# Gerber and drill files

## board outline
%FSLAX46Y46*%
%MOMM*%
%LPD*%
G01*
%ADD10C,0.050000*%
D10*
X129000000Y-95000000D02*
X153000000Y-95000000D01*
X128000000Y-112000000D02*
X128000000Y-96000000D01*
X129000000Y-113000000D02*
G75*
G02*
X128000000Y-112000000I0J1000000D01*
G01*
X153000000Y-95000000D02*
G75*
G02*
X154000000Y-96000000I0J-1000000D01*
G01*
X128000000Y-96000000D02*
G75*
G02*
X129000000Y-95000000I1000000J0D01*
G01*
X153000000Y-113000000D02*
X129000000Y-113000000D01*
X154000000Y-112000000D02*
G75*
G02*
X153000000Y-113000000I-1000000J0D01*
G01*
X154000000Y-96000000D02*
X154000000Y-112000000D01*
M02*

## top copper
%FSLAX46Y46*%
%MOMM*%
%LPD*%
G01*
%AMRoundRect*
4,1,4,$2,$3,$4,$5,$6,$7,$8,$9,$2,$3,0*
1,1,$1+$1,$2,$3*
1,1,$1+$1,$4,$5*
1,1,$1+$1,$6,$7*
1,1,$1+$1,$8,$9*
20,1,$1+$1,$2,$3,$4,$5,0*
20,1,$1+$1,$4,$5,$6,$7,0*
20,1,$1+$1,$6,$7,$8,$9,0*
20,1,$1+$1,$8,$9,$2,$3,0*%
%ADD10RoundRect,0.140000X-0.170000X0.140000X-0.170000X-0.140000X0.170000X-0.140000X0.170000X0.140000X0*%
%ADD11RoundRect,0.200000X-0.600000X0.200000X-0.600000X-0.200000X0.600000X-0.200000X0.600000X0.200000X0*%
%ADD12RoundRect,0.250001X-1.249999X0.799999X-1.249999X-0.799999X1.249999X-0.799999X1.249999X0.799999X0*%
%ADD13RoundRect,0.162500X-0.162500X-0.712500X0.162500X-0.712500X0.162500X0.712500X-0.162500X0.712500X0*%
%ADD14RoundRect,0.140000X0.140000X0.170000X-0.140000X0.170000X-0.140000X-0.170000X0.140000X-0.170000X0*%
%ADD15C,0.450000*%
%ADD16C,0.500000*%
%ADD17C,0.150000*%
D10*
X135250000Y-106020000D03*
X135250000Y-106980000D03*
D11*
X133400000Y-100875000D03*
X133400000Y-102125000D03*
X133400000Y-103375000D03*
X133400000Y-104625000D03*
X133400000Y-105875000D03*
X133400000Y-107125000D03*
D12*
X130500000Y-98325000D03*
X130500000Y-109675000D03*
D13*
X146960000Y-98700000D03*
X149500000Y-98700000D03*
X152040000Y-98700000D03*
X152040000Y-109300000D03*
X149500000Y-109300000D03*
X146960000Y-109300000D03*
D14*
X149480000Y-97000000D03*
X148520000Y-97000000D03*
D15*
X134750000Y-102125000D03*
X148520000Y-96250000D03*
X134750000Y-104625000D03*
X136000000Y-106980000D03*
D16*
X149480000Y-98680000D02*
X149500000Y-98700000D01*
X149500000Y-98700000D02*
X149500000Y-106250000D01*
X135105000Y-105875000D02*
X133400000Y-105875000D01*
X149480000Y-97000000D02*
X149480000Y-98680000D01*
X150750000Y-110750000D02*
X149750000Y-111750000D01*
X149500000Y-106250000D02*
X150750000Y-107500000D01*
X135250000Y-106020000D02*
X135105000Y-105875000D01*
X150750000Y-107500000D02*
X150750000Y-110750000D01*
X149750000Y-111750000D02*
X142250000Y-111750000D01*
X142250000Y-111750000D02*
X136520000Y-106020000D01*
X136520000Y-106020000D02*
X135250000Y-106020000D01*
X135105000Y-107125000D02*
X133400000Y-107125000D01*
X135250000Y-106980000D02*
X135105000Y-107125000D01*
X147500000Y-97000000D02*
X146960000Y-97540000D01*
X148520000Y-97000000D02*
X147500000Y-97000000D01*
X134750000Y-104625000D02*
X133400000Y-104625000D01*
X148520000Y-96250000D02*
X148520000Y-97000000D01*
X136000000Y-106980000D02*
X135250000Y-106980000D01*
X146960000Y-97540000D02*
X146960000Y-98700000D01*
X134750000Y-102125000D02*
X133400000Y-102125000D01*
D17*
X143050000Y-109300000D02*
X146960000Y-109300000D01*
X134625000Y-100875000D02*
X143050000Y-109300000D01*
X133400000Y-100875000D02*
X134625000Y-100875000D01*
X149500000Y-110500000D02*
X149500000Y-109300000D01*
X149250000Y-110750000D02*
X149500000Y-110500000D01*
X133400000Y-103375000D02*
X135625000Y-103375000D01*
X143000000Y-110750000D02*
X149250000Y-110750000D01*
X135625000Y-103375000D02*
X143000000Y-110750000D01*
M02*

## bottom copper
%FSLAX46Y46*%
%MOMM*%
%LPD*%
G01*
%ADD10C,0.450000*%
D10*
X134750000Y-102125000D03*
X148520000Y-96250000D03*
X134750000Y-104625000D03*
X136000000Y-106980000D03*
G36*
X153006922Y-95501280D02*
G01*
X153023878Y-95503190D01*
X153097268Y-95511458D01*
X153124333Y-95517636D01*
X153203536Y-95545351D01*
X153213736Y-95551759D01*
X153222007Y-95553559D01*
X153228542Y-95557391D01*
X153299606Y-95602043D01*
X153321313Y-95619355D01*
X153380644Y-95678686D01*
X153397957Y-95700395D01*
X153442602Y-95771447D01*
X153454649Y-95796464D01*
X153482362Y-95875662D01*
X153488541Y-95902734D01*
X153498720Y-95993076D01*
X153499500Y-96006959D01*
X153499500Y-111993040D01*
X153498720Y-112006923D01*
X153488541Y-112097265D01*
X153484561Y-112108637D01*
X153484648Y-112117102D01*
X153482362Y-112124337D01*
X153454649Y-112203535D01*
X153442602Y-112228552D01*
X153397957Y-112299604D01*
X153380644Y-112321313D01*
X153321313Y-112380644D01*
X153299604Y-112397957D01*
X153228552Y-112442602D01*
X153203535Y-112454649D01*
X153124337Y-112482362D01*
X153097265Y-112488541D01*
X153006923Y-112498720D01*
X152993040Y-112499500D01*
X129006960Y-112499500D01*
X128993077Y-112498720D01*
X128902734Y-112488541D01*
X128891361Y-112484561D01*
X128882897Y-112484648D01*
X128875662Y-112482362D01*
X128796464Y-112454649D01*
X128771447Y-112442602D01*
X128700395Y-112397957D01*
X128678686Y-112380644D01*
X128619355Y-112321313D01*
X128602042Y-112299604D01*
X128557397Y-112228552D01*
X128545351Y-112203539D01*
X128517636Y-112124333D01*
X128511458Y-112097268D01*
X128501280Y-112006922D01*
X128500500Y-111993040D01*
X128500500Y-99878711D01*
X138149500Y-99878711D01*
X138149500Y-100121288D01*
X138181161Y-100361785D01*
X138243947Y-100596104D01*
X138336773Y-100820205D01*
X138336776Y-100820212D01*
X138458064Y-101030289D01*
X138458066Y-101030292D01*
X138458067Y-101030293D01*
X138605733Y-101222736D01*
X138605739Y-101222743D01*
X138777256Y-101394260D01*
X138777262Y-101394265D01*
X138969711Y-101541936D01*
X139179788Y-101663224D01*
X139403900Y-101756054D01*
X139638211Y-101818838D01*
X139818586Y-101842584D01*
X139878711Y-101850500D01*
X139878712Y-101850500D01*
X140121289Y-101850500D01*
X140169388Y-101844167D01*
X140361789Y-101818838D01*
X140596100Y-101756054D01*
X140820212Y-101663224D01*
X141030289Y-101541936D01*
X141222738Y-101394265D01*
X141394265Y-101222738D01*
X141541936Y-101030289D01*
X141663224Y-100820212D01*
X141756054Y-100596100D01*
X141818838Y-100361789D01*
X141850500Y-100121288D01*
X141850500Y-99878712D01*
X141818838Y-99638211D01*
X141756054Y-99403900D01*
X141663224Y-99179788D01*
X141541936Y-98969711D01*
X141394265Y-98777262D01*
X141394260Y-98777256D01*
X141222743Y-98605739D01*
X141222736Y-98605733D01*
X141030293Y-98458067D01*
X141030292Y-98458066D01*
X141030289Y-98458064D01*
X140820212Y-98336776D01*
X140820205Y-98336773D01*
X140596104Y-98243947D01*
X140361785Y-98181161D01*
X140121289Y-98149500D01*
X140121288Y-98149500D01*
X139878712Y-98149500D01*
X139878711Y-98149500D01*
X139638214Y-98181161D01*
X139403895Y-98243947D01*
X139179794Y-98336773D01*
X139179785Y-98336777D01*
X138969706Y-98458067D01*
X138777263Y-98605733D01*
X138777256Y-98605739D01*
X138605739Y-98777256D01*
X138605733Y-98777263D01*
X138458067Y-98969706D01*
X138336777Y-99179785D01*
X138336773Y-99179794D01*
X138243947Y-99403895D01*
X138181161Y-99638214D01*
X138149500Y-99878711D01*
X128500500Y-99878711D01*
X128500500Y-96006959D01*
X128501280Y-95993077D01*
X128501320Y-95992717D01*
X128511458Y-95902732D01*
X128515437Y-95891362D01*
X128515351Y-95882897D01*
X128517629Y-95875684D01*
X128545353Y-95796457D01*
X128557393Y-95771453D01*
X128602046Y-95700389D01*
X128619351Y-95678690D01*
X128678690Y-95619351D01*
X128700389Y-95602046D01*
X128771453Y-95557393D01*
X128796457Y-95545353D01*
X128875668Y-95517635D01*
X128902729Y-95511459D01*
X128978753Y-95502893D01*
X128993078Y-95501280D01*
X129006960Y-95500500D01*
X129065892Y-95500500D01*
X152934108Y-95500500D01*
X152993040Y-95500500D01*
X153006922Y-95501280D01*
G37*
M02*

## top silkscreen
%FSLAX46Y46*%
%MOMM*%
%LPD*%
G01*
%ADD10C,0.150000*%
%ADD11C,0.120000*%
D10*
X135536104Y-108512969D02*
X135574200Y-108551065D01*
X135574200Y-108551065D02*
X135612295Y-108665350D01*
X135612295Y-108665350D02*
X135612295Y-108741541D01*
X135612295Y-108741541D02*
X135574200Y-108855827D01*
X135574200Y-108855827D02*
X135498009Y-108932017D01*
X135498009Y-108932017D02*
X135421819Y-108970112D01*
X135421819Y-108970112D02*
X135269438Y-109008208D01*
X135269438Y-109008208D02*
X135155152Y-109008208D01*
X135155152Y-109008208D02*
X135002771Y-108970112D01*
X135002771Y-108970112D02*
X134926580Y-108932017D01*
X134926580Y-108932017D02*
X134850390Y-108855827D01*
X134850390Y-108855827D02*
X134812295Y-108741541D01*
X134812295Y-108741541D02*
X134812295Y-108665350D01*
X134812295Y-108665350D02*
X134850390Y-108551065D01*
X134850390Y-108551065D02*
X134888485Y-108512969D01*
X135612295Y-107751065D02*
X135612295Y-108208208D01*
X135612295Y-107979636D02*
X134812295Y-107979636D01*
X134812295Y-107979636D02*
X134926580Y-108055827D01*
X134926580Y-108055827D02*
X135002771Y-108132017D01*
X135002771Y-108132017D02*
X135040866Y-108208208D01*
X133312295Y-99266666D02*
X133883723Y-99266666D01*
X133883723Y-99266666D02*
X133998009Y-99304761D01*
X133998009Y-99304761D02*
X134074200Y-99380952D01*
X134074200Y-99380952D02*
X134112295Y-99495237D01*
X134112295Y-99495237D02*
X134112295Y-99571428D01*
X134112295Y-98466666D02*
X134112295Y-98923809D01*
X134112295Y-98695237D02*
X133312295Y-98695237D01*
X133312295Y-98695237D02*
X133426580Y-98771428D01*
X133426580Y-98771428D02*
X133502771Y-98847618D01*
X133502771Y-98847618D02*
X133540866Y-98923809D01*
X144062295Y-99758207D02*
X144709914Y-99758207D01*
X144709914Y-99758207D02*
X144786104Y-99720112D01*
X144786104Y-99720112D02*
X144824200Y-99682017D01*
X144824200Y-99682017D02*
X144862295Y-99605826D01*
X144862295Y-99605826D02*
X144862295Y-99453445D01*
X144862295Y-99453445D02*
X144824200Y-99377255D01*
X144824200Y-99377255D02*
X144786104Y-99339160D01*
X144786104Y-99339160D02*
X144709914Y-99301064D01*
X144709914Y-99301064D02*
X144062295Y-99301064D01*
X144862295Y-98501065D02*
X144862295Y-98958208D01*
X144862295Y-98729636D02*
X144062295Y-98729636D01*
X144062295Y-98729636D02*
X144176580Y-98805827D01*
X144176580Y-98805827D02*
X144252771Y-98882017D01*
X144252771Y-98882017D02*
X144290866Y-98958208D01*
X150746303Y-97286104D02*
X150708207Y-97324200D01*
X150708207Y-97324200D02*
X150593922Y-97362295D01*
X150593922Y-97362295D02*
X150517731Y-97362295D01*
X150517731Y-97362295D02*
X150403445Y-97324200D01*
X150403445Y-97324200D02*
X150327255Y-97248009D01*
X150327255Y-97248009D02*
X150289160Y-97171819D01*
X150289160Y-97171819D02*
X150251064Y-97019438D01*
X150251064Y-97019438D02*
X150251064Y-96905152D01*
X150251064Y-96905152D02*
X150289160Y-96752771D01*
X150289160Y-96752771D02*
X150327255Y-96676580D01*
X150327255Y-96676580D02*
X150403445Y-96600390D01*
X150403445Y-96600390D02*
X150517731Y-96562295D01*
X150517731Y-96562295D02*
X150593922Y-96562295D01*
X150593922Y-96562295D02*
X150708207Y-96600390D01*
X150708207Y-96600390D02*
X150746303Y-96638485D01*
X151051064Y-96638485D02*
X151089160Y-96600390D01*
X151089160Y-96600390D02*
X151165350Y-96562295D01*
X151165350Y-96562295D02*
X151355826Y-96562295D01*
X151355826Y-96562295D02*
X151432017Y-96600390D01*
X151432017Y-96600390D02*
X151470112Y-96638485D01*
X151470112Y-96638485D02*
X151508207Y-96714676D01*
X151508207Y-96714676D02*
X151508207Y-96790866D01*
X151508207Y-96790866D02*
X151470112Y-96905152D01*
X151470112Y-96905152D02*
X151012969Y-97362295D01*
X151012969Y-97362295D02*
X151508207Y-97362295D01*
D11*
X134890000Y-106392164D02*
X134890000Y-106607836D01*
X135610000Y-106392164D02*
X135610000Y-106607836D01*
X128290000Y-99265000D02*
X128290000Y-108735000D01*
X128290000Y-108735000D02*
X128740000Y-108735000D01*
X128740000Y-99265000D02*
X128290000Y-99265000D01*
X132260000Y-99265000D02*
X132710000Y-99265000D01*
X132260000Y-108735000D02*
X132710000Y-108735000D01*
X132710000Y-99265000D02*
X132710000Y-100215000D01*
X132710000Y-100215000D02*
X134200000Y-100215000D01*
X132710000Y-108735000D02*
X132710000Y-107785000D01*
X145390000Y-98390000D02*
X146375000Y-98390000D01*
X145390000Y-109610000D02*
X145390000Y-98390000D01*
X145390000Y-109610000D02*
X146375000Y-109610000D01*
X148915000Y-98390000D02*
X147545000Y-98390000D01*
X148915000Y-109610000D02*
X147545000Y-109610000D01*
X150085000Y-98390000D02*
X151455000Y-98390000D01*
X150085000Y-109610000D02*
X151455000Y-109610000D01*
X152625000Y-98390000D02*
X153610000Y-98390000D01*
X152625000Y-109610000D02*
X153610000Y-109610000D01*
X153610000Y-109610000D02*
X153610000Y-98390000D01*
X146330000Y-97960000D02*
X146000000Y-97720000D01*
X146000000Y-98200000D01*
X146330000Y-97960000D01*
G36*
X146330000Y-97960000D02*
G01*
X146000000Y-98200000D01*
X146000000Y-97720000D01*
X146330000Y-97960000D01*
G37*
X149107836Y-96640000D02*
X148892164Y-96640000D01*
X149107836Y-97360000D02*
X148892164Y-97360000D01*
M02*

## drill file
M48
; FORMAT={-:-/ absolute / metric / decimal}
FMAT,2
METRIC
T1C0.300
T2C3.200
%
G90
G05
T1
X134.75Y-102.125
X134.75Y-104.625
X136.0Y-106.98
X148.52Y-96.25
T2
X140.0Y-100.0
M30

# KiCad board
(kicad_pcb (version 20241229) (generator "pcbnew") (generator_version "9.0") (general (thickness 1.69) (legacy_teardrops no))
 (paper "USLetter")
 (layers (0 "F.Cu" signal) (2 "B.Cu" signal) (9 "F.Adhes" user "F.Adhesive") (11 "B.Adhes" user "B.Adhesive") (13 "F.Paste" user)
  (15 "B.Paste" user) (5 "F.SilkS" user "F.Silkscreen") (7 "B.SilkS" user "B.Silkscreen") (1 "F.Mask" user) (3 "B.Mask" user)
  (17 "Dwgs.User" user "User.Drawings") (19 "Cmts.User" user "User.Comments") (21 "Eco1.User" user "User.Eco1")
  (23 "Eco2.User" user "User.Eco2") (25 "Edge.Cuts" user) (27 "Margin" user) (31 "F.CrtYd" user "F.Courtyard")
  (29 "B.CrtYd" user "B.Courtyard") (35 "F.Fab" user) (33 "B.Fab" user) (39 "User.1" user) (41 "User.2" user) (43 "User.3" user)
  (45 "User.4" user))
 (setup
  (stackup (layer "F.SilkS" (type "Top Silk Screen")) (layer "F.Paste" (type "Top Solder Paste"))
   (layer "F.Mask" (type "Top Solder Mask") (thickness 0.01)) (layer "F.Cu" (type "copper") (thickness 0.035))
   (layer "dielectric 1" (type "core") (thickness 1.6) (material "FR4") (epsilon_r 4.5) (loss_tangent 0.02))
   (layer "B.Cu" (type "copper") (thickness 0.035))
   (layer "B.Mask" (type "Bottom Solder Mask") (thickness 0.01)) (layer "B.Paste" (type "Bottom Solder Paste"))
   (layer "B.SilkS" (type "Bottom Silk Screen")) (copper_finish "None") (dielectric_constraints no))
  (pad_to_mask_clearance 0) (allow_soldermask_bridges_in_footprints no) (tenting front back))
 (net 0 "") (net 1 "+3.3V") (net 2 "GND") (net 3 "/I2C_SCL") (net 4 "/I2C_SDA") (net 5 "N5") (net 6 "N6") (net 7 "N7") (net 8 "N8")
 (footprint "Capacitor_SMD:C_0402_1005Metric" (layer "F.Cu") (at 135.25 106.5 -90)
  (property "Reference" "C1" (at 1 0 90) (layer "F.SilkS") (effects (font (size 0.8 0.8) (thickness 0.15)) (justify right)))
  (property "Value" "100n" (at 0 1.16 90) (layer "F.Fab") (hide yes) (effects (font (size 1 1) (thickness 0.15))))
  (fp_line (start -0.107836 0.36) (end 0.107836 0.36) (stroke (width 0.12) (type solid)) (layer "F.SilkS"))
  (fp_line (start -0.107836 -0.36) (end 0.107836 -0.36) (stroke (width 0.12) (type solid)) (layer "F.SilkS"))
  (pad "1" smd roundrect (at -0.48 0 270) (size 0.56 0.62) (layers "F.Cu" "F.Mask" "F.Paste") (roundrect_rratio 0.25) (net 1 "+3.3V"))
  (pad "2" smd roundrect (at 0.48 0 270) (size 0.56 0.62) (layers "F.Cu" "F.Mask" "F.Paste") (roundrect_rratio 0.25) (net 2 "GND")))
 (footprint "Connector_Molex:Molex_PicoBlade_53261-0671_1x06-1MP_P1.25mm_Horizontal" (layer "F.Cu") (at 131 104 -90)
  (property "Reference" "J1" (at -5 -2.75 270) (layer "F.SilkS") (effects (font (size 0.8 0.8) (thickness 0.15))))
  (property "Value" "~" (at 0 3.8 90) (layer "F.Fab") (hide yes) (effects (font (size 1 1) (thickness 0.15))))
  (fp_line (start -4.735 2.71) (end 4.735 2.71) (stroke (width 0.12) (type solid)) (layer "F.SilkS"))
  (fp_line (start 4.735 2.71) (end 4.735 2.26) (stroke (width 0.12) (type solid)) (layer "F.SilkS"))
  (fp_line (start -4.735 2.26) (end -4.735 2.71) (stroke (width 0.12) (type solid)) (layer "F.SilkS"))
  (fp_line (start -4.735 -1.26) (end -4.735 -1.71) (stroke (width 0.12) (type solid)) (layer "F.SilkS"))
  (fp_line (start 4.735 -1.26) (end 4.735 -1.71) (stroke (width 0.12) (type solid)) (layer "F.SilkS"))
  (fp_line (start -4.735 -1.71) (end -3.785 -1.71) (stroke (width 0.12) (type solid)) (layer "F.SilkS"))
  (fp_line (start -3.785 -1.71) (end -3.785 -3.2) (stroke (width 0.12) (type solid)) (layer "F.SilkS"))
  (fp_line (start 4.735 -1.71) (end 3.785 -1.71) (stroke (width 0.12) (type solid)) (layer "F.SilkS"))
  (pad "1" smd roundrect (at -3.125 -2.4 270) (size 0.8 1.6) (layers "F.Cu" "F.Mask" "F.Paste") (roundrect_rratio 0.25) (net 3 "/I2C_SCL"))
  (pad "2" smd roundrect (at -1.875 -2.4 270) (size 0.8 1.6) (layers "F.Cu" "F.Mask" "F.Paste") (roundrect_rratio 0.25) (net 2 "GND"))
  (pad "3" smd roundrect (at -0.625 -2.4 270) (size 0.8 1.6) (layers "F.Cu" "F.Mask" "F.Paste") (roundrect_rratio 0.25) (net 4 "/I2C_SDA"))
  (pad "4" smd roundrect (at 0.625 -2.4 270) (size 0.8 1.6) (layers "F.Cu" "F.Mask" "F.Paste") (roundrect_rratio 0.25) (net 2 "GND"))
  (pad "5" smd roundrect (at 1.875 -2.4 270) (size 0.8 1.6) (layers "F.Cu" "F.Mask" "F.Paste") (roundrect_rratio 0.25) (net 1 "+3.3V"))
  (pad "6" smd roundrect (at 3.125 -2.4 270) (size 0.8 1.6) (layers "F.Cu" "F.Mask" "F.Paste") (roundrect_rratio 0.25) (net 2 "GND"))
  (pad "MP" smd roundrect (at -5.675 0.5 270) (size 2.1 3) (layers "F.Cu" "F.Mask" "F.Paste") (roundrect_rratio 0.119048) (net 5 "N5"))
  (pad "MP" smd roundrect (at 5.675 0.5 270) (size 2.1 3) (layers "F.Cu" "F.Mask" "F.Paste") (roundrect_rratio 0.119048) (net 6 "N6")))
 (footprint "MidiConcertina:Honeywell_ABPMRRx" (layer "F.Cu") (at 149.5 104)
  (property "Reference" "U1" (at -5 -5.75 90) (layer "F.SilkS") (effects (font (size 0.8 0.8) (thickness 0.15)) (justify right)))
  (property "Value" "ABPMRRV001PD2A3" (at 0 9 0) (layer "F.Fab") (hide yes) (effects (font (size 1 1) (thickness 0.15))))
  (fp_line (start -4.11 -5.61) (end -3.125 -5.61) (stroke (width 0.12) (type solid)) (layer "F.SilkS"))
  (fp_line (start -4.11 5.61) (end -4.11 -5.61) (stroke (width 0.12) (type solid)) (layer "F.SilkS"))
  (fp_line (start -4.11 5.61) (end -3.125 5.61) (stroke (width 0.12) (type solid)) (layer "F.SilkS"))
  (fp_line (start -0.585 -5.61) (end -1.955 -5.61) (stroke (width 0.12) (type solid)) (layer "F.SilkS"))
  (fp_line (start -0.585 5.61) (end -1.955 5.61) (stroke (width 0.12) (type solid)) (layer "F.SilkS"))
  (fp_line (start 0.585 -5.61) (end 1.955 -5.61) (stroke (width 0.12) (type solid)) (layer "F.SilkS"))
  (fp_line (start 0.585 5.61) (end 1.955 5.61) (stroke (width 0.12) (type solid)) (layer "F.SilkS"))
  (fp_line (start 3.125 -5.61) (end 4.11 -5.61) (stroke (width 0.12) (type solid)) (layer "F.SilkS"))
  (fp_line (start 3.125 5.61) (end 4.11 5.61) (stroke (width 0.12) (type solid)) (layer "F.SilkS"))
  (fp_line (start 4.11 5.61) (end 4.11 -5.61) (stroke (width 0.12) (type solid)) (layer "F.SilkS"))
  (fp_poly
   (pts (xy -3.17 -6.04) (xy -3.5 -6.28) (xy -3.5 -5.8) (xy -3.17 -6.04)) (stroke (width 0.12) (type solid)) (fill yes) (layer "F.SilkS"))
  (pad "1" smd roundrect (at -2.54 -5.3) (size 0.65 1.75) (layers "F.Cu" "F.Mask" "F.Paste") (roundrect_rratio 0.25) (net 2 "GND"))
  (pad "2" smd roundrect (at 0 -5.3) (size 0.65 1.75) (layers "F.Cu" "F.Mask" "F.Paste") (roundrect_rratio 0.25) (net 1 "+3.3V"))
  (pad "3" smd roundrect (at 2.54 -5.3) (size 0.65 1.75) (layers "F.Cu" "F.Mask" "F.Paste") (roundrect_rratio 0.25) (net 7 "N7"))
  (pad "4" smd roundrect (at 2.54 5.3) (size 0.65 1.75) (layers "F.Cu" "F.Mask" "F.Paste") (roundrect_rratio 0.25) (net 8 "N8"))
  (pad "5" smd roundrect (at 0 5.3) (size 0.65 1.75) (layers "F.Cu" "F.Mask" "F.Paste") (roundrect_rratio 0.25) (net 4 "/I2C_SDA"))
  (pad "6" smd roundrect (at -2.54 5.3) (size 0.65 1.75) (layers "F.Cu" "F.Mask" "F.Paste") (roundrect_rratio 0.25) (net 3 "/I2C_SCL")))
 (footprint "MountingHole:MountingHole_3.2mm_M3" (layer "F.Cu") (at 140 100)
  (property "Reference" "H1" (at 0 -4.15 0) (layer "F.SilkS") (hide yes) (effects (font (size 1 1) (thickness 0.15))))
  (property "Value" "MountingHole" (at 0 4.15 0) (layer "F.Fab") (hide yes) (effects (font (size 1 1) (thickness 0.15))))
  (pad "" np_thru_hole circle (at 0 0) (size 3.2 3.2) (drill 3.2) (layers "*.Cu" "*.Mask")))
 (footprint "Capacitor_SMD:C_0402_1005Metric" (layer "F.Cu") (at 149 97 180)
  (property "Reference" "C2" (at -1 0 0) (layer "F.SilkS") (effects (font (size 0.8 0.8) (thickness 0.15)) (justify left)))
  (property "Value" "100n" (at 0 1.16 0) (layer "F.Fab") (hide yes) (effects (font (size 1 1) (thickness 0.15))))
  (fp_line (start -0.107836 0.36) (end 0.107836 0.36) (stroke (width 0.12) (type solid)) (layer "F.SilkS"))
  (fp_line (start -0.107836 -0.36) (end 0.107836 -0.36) (stroke (width 0.12) (type solid)) (layer "F.SilkS"))
  (pad "1" smd roundrect (at -0.48 0 180) (size 0.56 0.62) (layers "F.Cu" "F.Mask" "F.Paste") (roundrect_rratio 0.25) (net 1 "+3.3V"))
  (pad "2" smd roundrect (at 0.48 0 180) (size 0.56 0.62) (layers "F.Cu" "F.Mask" "F.Paste") (roundrect_rratio 0.25) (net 2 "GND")))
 (gr_line (start 129 95) (end 153 95) (stroke (width 0.05) (type default)) (layer "Edge.Cuts"))
 (gr_line (start 128 112) (end 128 96) (stroke (width 0.05) (type default)) (layer "Edge.Cuts"))
 (gr_arc (start 129 113) (mid 128.292893 112.707107) (end 128 112) (stroke (width 0.05) (type default)) (layer "Edge.Cuts"))
 (gr_arc (start 153 95) (mid 153.707107 95.292893) (end 154 96) (stroke (width 0.05) (type default)) (layer "Edge.Cuts"))
 (gr_arc (start 128 96) (mid 128.292893 95.292893) (end 129 95) (stroke (width 0.05) (type default)) (layer "Edge.Cuts"))
 (gr_line (start 153 113) (end 129 113) (stroke (width 0.05) (type default)) (layer "Edge.Cuts"))
 (gr_arc (start 154 112) (mid 153.707107 112.707107) (end 153 113) (stroke (width 0.05) (type default)) (layer "Edge.Cuts"))
 (gr_line (start 154 96) (end 154 112) (stroke (width 0.05) (type default)) (layer "Edge.Cuts"))
 (segment (start 149.48 98.68) (end 149.5 98.7) (width 0.5) (layer "F.Cu") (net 1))
 (segment (start 149.5 98.7) (end 149.5 106.25) (width 0.5) (layer "F.Cu") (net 1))
 (segment (start 135.105 105.875) (end 133.4 105.875) (width 0.5) (layer "F.Cu") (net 1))
 (segment (start 149.48 97) (end 149.48 98.68) (width 0.5) (layer "F.Cu") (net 1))
 (segment (start 150.75 110.75) (end 149.75 111.75) (width 0.5) (layer "F.Cu") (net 1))
 (segment (start 149.5 106.25) (end 150.75 107.5) (width 0.5) (layer "F.Cu") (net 1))
 (segment (start 135.25 106.02) (end 135.105 105.875) (width 0.5) (layer "F.Cu") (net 1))
 (segment (start 150.75 107.5) (end 150.75 110.75) (width 0.5) (layer "F.Cu") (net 1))
 (segment (start 149.75 111.75) (end 142.25 111.75) (width 0.5) (layer "F.Cu") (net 1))
 (segment (start 142.25 111.75) (end 136.52 106.02) (width 0.5) (layer "F.Cu") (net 1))
 (segment (start 136.52 106.02) (end 135.25 106.02) (width 0.5) (layer "F.Cu") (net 1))
 (segment (start 135.105 107.125) (end 133.4 107.125) (width 0.5) (layer "F.Cu") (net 2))
 (segment (start 135.25 106.98) (end 135.105 107.125) (width 0.5) (layer "F.Cu") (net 2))
 (segment (start 147.5 97) (end 146.96 97.54) (width 0.5) (layer "F.Cu") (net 2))
 (segment (start 148.52 97) (end 147.5 97) (width 0.5) (layer "F.Cu") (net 2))
 (segment (start 134.75 104.625) (end 133.4 104.625) (width 0.5) (layer "F.Cu") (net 2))
 (segment (start 148.52 96.25) (end 148.52 97) (width 0.5) (layer "F.Cu") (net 2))
 (segment (start 136 106.98) (end 135.25 106.98) (width 0.5) (layer "F.Cu") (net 2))
 (segment (start 146.96 97.54) (end 146.96 98.7) (width 0.5) (layer "F.Cu") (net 2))
 (segment (start 134.75 102.125) (end 133.4 102.125) (width 0.5) (layer "F.Cu") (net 2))
 (via (at 134.75 102.125) (size 0.45) (drill 0.3) (layers "F.Cu" "B.Cu") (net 2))
 (via (at 148.52 96.25) (size 0.45) (drill 0.3) (layers "F.Cu" "B.Cu") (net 2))
 (via (at 134.75 104.625) (size 0.45) (drill 0.3) (layers "F.Cu" "B.Cu") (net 2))
 (via (at 136 106.98) (size 0.45) (drill 0.3) (layers "F.Cu" "B.Cu") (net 2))
 (segment (start 143.05 109.3) (end 146.96 109.3) (width 0.15) (layer "F.Cu") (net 3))
 (segment (start 134.625 100.875) (end 143.05 109.3) (width 0.15) (layer "F.Cu") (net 3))
 (segment (start 133.4 100.875) (end 134.625 100.875) (width 0.15) (layer "F.Cu") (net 3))
 (segment (start 149.5 110.5) (end 149.5 109.3) (width 0.15) (layer "F.Cu") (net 4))
 (segment (start 149.25 110.75) (end 149.5 110.5) (width 0.15) (layer "F.Cu") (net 4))
 (segment (start 133.4 103.375) (end 135.625 103.375) (width 0.15) (layer "F.Cu") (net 4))
 (segment (start 143 110.75) (end 149.25 110.75) (width 0.15) (layer "F.Cu") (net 4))
 (segment (start 135.625 103.375) (end 143 110.75) (width 0.15) (layer "F.Cu") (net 4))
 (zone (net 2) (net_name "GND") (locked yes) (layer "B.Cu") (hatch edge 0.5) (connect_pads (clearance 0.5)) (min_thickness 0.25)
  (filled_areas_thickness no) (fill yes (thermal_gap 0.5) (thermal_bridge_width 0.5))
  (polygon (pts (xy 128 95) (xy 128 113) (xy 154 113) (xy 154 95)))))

